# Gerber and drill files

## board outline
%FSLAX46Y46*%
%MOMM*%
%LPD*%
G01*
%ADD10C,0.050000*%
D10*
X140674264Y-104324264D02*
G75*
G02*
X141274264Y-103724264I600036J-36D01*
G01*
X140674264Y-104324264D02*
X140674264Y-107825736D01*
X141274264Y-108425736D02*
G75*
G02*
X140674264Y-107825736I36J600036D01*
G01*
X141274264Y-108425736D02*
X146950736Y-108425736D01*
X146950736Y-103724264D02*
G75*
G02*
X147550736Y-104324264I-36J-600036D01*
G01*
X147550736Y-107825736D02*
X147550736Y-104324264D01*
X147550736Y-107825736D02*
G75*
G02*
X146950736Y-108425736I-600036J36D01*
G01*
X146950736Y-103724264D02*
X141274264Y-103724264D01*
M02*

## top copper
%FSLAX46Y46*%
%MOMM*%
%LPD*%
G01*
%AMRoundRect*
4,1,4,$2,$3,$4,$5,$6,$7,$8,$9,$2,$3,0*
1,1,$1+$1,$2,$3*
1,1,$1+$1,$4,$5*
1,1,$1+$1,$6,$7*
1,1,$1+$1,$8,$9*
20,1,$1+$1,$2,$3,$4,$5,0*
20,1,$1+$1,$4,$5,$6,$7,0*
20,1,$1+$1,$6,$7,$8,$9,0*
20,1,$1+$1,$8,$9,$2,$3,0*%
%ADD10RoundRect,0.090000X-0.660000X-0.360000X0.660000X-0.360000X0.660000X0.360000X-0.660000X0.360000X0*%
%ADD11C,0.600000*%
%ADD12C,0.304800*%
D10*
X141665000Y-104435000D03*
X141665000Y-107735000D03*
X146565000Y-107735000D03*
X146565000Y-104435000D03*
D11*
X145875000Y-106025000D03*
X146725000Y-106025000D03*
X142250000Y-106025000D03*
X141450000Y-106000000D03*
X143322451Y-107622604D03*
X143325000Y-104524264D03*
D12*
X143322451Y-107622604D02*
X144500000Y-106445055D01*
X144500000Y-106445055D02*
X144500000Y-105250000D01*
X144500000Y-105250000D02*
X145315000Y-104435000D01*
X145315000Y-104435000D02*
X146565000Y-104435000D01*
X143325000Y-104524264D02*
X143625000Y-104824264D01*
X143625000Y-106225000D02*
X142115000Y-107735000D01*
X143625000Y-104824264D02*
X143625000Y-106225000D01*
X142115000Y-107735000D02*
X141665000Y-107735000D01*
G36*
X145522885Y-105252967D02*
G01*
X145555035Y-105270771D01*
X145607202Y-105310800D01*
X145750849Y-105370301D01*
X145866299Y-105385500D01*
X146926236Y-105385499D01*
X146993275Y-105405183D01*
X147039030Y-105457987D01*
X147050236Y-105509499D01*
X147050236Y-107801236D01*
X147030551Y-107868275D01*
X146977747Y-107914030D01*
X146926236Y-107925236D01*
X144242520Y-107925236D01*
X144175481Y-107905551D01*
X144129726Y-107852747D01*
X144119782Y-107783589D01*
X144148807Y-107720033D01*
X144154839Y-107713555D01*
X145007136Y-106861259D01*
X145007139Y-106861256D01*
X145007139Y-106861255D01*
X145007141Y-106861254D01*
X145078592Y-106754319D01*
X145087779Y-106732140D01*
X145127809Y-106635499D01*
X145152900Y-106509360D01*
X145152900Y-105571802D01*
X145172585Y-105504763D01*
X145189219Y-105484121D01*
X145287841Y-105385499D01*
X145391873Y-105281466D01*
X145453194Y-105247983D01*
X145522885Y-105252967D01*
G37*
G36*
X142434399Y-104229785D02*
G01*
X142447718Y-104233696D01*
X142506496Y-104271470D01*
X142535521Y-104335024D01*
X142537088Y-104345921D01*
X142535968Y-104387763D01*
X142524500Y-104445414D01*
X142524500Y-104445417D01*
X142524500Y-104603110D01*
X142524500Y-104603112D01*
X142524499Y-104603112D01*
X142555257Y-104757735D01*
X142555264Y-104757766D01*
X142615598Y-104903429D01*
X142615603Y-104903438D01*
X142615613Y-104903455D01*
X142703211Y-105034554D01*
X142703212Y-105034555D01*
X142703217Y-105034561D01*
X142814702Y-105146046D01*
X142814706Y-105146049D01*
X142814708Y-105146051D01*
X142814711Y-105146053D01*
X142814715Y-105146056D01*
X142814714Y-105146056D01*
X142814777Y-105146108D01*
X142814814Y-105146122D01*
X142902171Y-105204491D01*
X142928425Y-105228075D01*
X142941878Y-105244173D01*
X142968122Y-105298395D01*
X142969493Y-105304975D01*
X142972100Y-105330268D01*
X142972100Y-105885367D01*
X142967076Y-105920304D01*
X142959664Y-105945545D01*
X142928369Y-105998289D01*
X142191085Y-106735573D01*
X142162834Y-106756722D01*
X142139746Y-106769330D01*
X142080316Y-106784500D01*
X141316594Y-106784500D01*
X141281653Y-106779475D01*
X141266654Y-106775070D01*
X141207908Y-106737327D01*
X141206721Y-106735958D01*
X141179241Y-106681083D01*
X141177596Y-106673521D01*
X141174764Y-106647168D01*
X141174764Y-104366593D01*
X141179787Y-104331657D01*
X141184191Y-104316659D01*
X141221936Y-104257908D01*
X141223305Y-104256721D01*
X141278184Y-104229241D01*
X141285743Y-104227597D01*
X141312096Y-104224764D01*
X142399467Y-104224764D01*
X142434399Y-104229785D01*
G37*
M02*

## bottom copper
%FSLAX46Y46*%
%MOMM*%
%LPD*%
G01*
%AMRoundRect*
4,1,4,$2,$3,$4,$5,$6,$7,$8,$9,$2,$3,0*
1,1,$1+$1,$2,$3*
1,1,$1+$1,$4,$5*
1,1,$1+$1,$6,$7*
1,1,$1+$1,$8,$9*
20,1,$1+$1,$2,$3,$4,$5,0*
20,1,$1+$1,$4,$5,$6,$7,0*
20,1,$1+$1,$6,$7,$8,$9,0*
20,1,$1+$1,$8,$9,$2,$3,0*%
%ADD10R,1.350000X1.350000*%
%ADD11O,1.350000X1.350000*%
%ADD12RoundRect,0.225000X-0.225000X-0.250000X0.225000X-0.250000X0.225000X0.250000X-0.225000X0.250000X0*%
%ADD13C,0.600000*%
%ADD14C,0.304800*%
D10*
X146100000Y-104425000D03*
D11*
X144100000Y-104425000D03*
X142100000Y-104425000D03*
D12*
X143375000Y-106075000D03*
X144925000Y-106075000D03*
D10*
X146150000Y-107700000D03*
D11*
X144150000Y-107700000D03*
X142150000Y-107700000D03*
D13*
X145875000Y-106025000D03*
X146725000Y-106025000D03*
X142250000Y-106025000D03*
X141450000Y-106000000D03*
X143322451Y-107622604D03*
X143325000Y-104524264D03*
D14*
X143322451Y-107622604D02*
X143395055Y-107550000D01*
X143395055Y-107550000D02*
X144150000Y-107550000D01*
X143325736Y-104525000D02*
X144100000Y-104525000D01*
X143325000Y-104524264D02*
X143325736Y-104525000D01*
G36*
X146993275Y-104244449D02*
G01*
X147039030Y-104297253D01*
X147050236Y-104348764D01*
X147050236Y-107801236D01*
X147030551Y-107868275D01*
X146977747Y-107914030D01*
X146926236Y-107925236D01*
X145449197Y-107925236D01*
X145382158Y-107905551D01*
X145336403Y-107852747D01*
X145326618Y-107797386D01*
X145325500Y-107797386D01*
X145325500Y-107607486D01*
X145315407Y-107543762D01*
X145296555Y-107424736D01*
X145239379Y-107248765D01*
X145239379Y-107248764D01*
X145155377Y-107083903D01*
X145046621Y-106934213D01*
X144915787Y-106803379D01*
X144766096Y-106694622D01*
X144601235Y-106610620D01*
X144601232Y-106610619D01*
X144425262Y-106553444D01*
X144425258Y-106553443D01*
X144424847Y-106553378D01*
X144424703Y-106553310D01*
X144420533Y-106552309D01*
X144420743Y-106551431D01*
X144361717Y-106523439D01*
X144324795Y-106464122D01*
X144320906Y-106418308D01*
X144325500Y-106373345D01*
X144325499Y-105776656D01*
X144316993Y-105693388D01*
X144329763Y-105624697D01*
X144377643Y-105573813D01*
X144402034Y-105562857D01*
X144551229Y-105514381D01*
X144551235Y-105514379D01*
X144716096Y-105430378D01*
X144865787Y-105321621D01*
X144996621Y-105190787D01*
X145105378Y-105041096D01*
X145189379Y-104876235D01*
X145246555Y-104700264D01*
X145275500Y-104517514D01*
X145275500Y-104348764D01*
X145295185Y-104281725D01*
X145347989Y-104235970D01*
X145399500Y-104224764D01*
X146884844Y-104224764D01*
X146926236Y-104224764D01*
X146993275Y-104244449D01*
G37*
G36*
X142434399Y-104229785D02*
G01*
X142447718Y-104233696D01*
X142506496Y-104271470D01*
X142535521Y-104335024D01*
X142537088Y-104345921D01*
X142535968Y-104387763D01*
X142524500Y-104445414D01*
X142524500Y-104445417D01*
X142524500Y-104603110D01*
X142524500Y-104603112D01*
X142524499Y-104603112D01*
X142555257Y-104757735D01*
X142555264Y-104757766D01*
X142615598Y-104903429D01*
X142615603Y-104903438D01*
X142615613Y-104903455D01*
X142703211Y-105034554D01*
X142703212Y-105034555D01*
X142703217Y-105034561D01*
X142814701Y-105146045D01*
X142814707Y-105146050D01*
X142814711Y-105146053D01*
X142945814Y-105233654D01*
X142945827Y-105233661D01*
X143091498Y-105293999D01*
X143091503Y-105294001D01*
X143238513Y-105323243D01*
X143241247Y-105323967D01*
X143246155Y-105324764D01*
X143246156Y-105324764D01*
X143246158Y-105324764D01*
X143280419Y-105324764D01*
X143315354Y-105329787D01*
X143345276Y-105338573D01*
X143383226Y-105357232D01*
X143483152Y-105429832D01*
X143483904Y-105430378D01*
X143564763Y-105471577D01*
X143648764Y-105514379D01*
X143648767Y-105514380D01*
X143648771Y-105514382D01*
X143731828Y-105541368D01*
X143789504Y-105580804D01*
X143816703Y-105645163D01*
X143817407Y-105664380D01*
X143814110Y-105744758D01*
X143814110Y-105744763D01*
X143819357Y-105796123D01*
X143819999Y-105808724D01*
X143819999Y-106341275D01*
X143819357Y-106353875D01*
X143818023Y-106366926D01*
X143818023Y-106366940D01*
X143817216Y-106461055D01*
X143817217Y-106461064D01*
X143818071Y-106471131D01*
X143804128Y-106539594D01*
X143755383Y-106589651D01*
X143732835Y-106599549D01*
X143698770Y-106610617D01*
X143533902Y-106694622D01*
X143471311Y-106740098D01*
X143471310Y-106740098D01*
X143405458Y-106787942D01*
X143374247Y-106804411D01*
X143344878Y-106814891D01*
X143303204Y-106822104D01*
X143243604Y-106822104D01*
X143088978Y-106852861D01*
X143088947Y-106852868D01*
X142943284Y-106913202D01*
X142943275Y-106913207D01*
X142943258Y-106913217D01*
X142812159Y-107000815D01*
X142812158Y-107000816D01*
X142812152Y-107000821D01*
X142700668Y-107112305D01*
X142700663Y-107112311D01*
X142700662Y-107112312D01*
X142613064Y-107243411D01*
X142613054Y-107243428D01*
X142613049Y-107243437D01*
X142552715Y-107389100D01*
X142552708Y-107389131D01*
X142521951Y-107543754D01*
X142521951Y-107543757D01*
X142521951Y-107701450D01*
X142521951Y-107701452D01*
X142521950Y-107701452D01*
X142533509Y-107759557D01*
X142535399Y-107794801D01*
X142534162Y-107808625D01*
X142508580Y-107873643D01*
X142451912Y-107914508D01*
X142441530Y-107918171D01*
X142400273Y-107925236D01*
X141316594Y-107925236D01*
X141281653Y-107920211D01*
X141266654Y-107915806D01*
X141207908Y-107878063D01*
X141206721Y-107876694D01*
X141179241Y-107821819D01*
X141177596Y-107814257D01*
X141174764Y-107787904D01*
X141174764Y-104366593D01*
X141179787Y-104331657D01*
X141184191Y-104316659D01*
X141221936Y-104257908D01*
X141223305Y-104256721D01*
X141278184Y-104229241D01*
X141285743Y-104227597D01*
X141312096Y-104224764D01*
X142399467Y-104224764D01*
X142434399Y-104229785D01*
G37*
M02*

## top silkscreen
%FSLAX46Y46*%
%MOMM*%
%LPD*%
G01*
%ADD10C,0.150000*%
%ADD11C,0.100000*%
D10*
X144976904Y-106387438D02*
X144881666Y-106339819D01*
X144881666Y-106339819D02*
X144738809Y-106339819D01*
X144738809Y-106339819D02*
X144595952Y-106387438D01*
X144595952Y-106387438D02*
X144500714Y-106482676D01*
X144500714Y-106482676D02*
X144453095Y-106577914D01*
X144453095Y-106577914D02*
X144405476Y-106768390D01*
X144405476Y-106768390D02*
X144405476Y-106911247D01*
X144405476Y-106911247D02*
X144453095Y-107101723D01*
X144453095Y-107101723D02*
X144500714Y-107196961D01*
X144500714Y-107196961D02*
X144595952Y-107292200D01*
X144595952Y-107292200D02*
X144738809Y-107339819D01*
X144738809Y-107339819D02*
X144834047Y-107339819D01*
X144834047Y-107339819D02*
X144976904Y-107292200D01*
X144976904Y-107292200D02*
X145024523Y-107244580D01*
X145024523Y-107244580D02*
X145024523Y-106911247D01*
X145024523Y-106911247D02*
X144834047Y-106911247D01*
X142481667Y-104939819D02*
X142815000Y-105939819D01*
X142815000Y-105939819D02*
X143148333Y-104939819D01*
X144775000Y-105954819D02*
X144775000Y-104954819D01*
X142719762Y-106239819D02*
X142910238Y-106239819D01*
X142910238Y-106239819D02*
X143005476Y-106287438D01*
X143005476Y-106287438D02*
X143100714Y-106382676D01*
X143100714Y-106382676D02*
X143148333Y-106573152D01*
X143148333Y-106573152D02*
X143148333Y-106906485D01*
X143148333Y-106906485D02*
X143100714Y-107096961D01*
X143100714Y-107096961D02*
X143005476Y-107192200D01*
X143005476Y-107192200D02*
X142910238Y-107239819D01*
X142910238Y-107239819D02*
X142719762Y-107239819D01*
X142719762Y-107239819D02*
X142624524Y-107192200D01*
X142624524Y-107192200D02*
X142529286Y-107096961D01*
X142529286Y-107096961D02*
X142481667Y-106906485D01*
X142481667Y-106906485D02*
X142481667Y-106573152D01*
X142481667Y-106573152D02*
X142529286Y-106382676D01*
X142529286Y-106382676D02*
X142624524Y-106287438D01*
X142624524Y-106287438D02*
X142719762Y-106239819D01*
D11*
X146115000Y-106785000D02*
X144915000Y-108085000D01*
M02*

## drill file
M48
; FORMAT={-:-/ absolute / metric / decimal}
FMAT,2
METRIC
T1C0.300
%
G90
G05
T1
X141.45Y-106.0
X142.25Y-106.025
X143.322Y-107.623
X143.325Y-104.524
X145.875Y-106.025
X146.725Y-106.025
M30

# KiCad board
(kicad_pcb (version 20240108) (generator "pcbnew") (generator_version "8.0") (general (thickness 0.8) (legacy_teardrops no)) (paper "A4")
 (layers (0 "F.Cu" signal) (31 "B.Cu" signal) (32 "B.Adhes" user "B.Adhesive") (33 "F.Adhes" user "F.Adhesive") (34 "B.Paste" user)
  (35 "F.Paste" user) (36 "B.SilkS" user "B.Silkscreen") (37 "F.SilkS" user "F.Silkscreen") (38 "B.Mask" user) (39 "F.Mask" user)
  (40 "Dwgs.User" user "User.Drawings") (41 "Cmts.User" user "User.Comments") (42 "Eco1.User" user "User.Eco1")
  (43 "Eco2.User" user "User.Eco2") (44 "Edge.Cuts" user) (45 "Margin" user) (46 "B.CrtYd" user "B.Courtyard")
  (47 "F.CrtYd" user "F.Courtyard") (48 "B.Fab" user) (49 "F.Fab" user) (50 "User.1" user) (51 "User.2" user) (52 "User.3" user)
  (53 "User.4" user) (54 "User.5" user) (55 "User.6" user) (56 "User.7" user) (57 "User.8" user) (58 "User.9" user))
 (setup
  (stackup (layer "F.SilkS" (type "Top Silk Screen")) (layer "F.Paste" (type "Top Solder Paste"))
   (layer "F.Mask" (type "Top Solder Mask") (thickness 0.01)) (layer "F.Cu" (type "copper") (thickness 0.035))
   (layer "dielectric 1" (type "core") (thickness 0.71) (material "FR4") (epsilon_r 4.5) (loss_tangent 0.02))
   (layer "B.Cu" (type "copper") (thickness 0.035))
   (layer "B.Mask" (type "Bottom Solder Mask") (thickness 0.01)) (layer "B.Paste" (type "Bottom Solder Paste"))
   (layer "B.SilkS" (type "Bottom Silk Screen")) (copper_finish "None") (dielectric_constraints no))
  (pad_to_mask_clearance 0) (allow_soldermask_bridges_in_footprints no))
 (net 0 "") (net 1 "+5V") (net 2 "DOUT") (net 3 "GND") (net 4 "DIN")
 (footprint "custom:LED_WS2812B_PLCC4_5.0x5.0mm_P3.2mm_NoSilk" (layer "F.Cu") (at 144.115 106.085)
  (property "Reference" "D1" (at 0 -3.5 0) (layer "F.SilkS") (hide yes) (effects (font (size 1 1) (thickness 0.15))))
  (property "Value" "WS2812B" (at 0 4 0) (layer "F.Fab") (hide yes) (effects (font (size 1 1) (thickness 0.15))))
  (fp_line (start 2 0.7) (end 0.8 2) (stroke (width 0.1) (type default)) (layer "F.SilkS"))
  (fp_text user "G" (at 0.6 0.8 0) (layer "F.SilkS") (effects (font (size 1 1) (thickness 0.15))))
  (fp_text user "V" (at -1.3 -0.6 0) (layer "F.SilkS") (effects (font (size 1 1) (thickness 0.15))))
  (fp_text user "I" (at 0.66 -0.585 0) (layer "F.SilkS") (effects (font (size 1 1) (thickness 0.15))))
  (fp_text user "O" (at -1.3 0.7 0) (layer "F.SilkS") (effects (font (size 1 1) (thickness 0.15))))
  (pad "1" smd roundrect (at -2.45 -1.65) (size 1.5 0.9) (layers "F.Cu" "F.Paste" "F.Mask") (roundrect_rratio 0.1) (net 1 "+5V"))
  (pad "2" smd roundrect (at -2.45 1.65) (size 1.5 0.9) (layers "F.Cu" "F.Paste" "F.Mask") (roundrect_rratio 0.1) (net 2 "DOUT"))
  (pad "3" smd roundrect (at 2.45 1.65) (size 1.5 0.9) (layers "F.Cu" "F.Paste" "F.Mask") (roundrect_rratio 0.1) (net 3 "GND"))
  (pad "4" smd roundrect (at 2.45 -1.65) (size 1.5 0.9) (layers "F.Cu" "F.Paste" "F.Mask") (roundrect_rratio 0.1) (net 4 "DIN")))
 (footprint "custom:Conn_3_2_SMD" (layer "B.Cu") (at 146.1 104.425 90)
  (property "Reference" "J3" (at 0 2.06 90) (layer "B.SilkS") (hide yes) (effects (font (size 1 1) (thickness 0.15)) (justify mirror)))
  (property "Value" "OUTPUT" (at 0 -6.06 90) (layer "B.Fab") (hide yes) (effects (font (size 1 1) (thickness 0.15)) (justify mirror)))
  (pad "1" smd rect (at 0 0 90) (size 1.35 1.35) (layers "B.Cu" "B.Paste" "B.Mask") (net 3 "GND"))
  (pad "2" smd oval (at 0 -2 90) (size 1.35 1.35) (layers "B.Cu" "B.Paste" "B.Mask") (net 2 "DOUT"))
  (pad "3" smd oval (at 0 -4 90) (size 1.35 1.35) (layers "B.Cu" "B.Paste" "B.Mask") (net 1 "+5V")))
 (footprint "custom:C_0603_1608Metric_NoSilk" (layer "B.Cu") (at 144.15 106.075)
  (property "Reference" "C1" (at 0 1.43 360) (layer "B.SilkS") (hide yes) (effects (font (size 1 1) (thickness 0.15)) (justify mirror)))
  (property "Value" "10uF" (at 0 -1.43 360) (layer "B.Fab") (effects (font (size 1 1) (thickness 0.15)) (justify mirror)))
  (pad "1" smd roundrect (at -0.775 0) (size 0.9 0.95) (layers "B.Cu" "B.Paste" "B.Mask") (roundrect_rratio 0.25) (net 1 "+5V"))
  (pad "2" smd roundrect (at 0.775 0) (size 0.9 0.95) (layers "B.Cu" "B.Paste" "B.Mask") (roundrect_rratio 0.25) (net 3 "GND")))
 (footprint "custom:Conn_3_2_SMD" (layer "B.Cu") (at 146.15 107.7 90)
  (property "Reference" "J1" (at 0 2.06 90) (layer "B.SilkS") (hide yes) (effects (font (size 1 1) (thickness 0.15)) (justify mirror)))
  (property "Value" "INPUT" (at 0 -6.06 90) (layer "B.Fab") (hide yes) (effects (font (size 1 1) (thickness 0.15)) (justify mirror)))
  (pad "1" smd rect (at 0 0 90) (size 1.35 1.35) (layers "B.Cu" "B.Paste" "B.Mask") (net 3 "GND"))
  (pad "2" smd oval (at 0 -2 90) (size 1.35 1.35) (layers "B.Cu" "B.Paste" "B.Mask") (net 4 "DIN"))
  (pad "3" smd oval (at 0 -4 90) (size 1.35 1.35) (layers "B.Cu" "B.Paste" "B.Mask") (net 1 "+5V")))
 (gr_arc (start 140.674264 104.324264) (mid 140.85 103.9) (end 141.274264 103.724264) (stroke (width 0.05) (type default))
  (layer "Edge.Cuts"))
 (gr_line (start 140.674264 104.324264) (end 140.674264 107.825736) (stroke (width 0.05) (type default)) (layer "Edge.Cuts"))
 (gr_arc (start 141.274264 108.425736) (mid 140.85 108.25) (end 140.674264 107.825736) (stroke (width 0.05) (type default))
  (layer "Edge.Cuts"))
 (gr_line (start 141.274264 108.425736) (end 146.950736 108.425736) (stroke (width 0.05) (type default)) (layer "Edge.Cuts"))
 (gr_arc (start 146.950736 103.724264) (mid 147.375 103.9) (end 147.550736 104.324264) (stroke (width 0.05) (type default))
  (layer "Edge.Cuts"))
 (gr_line (start 147.550736 107.825736) (end 147.550736 104.324264) (stroke (width 0.05) (type default)) (layer "Edge.Cuts"))
 (gr_arc (start 147.550736 107.825736) (mid 147.375 108.25) (end 146.950736 108.425736) (stroke (width 0.05) (type default))
  (layer "Edge.Cuts"))
 (gr_line (start 146.950736 103.724264) (end 141.274264 103.724264) (stroke (width 0.05) (type default)) (layer "Edge.Cuts"))
 (via (at 145.875 106.025) (size 0.6) (drill 0.3) (layers "F.Cu" "B.Cu") (free yes) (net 3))
 (via (at 146.725 106.025) (size 0.6) (drill 0.3) (layers "F.Cu" "B.Cu") (free yes) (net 3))
 (via (at 142.25 106.025) (size 0.6) (drill 0.3) (layers "F.Cu" "B.Cu") (free yes) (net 1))
 (via (at 141.45 106) (size 0.6) (drill 0.3) (layers "F.Cu" "B.Cu") (free yes) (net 1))
 (segment (start 143.322451 107.622604) (end 144.5 106.445055) (width 0.3048) (layer "F.Cu") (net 4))
 (segment (start 144.5 106.445055) (end 144.5 105.25) (width 0.3048) (layer "F.Cu") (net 4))
 (segment (start 144.5 105.25) (end 145.315 104.435) (width 0.3048) (layer "F.Cu") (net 4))
 (segment (start 145.315 104.435) (end 146.565 104.435) (width 0.3048) (layer "F.Cu") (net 4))
 (via (at 143.322451 107.622604) (size 0.6) (drill 0.3) (layers "F.Cu" "B.Cu") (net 4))
 (segment (start 143.322451 107.622604) (end 143.395055 107.55) (width 0.3048) (layer "B.Cu") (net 4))
 (segment (start 143.395055 107.55) (end 144.15 107.55) (width 0.3048) (layer "B.Cu") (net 4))
 (segment (start 143.325 104.524264) (end 143.625 104.824264) (width 0.3048) (layer "F.Cu") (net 2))
 (segment (start 143.625 106.225) (end 142.115 107.735) (width 0.3048) (layer "F.Cu") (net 2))
 (segment (start 143.625 104.824264) (end 143.625 106.225) (width 0.3048) (layer "F.Cu") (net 2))
 (segment (start 142.115 107.735) (end 141.665 107.735) (width 0.3048) (layer "F.Cu") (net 2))
 (via (at 143.325 104.524264) (size 0.6) (drill 0.3) (layers "F.Cu" "B.Cu") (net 2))
 (segment (start 143.325736 104.525) (end 144.1 104.525) (width 0.3048) (layer "B.Cu") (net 2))
 (segment (start 143.325 104.524264) (end 143.325736 104.525) (width 0.3048) (layer "B.Cu") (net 2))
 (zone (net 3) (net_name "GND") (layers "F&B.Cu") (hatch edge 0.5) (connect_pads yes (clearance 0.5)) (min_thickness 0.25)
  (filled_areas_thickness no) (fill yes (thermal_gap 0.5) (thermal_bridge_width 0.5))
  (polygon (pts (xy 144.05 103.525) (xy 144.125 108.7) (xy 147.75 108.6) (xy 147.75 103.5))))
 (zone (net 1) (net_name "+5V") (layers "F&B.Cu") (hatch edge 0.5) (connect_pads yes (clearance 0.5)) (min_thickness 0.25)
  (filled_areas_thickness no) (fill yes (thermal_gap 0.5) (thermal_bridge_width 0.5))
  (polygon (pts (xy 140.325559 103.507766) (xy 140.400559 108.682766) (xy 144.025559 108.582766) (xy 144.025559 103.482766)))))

